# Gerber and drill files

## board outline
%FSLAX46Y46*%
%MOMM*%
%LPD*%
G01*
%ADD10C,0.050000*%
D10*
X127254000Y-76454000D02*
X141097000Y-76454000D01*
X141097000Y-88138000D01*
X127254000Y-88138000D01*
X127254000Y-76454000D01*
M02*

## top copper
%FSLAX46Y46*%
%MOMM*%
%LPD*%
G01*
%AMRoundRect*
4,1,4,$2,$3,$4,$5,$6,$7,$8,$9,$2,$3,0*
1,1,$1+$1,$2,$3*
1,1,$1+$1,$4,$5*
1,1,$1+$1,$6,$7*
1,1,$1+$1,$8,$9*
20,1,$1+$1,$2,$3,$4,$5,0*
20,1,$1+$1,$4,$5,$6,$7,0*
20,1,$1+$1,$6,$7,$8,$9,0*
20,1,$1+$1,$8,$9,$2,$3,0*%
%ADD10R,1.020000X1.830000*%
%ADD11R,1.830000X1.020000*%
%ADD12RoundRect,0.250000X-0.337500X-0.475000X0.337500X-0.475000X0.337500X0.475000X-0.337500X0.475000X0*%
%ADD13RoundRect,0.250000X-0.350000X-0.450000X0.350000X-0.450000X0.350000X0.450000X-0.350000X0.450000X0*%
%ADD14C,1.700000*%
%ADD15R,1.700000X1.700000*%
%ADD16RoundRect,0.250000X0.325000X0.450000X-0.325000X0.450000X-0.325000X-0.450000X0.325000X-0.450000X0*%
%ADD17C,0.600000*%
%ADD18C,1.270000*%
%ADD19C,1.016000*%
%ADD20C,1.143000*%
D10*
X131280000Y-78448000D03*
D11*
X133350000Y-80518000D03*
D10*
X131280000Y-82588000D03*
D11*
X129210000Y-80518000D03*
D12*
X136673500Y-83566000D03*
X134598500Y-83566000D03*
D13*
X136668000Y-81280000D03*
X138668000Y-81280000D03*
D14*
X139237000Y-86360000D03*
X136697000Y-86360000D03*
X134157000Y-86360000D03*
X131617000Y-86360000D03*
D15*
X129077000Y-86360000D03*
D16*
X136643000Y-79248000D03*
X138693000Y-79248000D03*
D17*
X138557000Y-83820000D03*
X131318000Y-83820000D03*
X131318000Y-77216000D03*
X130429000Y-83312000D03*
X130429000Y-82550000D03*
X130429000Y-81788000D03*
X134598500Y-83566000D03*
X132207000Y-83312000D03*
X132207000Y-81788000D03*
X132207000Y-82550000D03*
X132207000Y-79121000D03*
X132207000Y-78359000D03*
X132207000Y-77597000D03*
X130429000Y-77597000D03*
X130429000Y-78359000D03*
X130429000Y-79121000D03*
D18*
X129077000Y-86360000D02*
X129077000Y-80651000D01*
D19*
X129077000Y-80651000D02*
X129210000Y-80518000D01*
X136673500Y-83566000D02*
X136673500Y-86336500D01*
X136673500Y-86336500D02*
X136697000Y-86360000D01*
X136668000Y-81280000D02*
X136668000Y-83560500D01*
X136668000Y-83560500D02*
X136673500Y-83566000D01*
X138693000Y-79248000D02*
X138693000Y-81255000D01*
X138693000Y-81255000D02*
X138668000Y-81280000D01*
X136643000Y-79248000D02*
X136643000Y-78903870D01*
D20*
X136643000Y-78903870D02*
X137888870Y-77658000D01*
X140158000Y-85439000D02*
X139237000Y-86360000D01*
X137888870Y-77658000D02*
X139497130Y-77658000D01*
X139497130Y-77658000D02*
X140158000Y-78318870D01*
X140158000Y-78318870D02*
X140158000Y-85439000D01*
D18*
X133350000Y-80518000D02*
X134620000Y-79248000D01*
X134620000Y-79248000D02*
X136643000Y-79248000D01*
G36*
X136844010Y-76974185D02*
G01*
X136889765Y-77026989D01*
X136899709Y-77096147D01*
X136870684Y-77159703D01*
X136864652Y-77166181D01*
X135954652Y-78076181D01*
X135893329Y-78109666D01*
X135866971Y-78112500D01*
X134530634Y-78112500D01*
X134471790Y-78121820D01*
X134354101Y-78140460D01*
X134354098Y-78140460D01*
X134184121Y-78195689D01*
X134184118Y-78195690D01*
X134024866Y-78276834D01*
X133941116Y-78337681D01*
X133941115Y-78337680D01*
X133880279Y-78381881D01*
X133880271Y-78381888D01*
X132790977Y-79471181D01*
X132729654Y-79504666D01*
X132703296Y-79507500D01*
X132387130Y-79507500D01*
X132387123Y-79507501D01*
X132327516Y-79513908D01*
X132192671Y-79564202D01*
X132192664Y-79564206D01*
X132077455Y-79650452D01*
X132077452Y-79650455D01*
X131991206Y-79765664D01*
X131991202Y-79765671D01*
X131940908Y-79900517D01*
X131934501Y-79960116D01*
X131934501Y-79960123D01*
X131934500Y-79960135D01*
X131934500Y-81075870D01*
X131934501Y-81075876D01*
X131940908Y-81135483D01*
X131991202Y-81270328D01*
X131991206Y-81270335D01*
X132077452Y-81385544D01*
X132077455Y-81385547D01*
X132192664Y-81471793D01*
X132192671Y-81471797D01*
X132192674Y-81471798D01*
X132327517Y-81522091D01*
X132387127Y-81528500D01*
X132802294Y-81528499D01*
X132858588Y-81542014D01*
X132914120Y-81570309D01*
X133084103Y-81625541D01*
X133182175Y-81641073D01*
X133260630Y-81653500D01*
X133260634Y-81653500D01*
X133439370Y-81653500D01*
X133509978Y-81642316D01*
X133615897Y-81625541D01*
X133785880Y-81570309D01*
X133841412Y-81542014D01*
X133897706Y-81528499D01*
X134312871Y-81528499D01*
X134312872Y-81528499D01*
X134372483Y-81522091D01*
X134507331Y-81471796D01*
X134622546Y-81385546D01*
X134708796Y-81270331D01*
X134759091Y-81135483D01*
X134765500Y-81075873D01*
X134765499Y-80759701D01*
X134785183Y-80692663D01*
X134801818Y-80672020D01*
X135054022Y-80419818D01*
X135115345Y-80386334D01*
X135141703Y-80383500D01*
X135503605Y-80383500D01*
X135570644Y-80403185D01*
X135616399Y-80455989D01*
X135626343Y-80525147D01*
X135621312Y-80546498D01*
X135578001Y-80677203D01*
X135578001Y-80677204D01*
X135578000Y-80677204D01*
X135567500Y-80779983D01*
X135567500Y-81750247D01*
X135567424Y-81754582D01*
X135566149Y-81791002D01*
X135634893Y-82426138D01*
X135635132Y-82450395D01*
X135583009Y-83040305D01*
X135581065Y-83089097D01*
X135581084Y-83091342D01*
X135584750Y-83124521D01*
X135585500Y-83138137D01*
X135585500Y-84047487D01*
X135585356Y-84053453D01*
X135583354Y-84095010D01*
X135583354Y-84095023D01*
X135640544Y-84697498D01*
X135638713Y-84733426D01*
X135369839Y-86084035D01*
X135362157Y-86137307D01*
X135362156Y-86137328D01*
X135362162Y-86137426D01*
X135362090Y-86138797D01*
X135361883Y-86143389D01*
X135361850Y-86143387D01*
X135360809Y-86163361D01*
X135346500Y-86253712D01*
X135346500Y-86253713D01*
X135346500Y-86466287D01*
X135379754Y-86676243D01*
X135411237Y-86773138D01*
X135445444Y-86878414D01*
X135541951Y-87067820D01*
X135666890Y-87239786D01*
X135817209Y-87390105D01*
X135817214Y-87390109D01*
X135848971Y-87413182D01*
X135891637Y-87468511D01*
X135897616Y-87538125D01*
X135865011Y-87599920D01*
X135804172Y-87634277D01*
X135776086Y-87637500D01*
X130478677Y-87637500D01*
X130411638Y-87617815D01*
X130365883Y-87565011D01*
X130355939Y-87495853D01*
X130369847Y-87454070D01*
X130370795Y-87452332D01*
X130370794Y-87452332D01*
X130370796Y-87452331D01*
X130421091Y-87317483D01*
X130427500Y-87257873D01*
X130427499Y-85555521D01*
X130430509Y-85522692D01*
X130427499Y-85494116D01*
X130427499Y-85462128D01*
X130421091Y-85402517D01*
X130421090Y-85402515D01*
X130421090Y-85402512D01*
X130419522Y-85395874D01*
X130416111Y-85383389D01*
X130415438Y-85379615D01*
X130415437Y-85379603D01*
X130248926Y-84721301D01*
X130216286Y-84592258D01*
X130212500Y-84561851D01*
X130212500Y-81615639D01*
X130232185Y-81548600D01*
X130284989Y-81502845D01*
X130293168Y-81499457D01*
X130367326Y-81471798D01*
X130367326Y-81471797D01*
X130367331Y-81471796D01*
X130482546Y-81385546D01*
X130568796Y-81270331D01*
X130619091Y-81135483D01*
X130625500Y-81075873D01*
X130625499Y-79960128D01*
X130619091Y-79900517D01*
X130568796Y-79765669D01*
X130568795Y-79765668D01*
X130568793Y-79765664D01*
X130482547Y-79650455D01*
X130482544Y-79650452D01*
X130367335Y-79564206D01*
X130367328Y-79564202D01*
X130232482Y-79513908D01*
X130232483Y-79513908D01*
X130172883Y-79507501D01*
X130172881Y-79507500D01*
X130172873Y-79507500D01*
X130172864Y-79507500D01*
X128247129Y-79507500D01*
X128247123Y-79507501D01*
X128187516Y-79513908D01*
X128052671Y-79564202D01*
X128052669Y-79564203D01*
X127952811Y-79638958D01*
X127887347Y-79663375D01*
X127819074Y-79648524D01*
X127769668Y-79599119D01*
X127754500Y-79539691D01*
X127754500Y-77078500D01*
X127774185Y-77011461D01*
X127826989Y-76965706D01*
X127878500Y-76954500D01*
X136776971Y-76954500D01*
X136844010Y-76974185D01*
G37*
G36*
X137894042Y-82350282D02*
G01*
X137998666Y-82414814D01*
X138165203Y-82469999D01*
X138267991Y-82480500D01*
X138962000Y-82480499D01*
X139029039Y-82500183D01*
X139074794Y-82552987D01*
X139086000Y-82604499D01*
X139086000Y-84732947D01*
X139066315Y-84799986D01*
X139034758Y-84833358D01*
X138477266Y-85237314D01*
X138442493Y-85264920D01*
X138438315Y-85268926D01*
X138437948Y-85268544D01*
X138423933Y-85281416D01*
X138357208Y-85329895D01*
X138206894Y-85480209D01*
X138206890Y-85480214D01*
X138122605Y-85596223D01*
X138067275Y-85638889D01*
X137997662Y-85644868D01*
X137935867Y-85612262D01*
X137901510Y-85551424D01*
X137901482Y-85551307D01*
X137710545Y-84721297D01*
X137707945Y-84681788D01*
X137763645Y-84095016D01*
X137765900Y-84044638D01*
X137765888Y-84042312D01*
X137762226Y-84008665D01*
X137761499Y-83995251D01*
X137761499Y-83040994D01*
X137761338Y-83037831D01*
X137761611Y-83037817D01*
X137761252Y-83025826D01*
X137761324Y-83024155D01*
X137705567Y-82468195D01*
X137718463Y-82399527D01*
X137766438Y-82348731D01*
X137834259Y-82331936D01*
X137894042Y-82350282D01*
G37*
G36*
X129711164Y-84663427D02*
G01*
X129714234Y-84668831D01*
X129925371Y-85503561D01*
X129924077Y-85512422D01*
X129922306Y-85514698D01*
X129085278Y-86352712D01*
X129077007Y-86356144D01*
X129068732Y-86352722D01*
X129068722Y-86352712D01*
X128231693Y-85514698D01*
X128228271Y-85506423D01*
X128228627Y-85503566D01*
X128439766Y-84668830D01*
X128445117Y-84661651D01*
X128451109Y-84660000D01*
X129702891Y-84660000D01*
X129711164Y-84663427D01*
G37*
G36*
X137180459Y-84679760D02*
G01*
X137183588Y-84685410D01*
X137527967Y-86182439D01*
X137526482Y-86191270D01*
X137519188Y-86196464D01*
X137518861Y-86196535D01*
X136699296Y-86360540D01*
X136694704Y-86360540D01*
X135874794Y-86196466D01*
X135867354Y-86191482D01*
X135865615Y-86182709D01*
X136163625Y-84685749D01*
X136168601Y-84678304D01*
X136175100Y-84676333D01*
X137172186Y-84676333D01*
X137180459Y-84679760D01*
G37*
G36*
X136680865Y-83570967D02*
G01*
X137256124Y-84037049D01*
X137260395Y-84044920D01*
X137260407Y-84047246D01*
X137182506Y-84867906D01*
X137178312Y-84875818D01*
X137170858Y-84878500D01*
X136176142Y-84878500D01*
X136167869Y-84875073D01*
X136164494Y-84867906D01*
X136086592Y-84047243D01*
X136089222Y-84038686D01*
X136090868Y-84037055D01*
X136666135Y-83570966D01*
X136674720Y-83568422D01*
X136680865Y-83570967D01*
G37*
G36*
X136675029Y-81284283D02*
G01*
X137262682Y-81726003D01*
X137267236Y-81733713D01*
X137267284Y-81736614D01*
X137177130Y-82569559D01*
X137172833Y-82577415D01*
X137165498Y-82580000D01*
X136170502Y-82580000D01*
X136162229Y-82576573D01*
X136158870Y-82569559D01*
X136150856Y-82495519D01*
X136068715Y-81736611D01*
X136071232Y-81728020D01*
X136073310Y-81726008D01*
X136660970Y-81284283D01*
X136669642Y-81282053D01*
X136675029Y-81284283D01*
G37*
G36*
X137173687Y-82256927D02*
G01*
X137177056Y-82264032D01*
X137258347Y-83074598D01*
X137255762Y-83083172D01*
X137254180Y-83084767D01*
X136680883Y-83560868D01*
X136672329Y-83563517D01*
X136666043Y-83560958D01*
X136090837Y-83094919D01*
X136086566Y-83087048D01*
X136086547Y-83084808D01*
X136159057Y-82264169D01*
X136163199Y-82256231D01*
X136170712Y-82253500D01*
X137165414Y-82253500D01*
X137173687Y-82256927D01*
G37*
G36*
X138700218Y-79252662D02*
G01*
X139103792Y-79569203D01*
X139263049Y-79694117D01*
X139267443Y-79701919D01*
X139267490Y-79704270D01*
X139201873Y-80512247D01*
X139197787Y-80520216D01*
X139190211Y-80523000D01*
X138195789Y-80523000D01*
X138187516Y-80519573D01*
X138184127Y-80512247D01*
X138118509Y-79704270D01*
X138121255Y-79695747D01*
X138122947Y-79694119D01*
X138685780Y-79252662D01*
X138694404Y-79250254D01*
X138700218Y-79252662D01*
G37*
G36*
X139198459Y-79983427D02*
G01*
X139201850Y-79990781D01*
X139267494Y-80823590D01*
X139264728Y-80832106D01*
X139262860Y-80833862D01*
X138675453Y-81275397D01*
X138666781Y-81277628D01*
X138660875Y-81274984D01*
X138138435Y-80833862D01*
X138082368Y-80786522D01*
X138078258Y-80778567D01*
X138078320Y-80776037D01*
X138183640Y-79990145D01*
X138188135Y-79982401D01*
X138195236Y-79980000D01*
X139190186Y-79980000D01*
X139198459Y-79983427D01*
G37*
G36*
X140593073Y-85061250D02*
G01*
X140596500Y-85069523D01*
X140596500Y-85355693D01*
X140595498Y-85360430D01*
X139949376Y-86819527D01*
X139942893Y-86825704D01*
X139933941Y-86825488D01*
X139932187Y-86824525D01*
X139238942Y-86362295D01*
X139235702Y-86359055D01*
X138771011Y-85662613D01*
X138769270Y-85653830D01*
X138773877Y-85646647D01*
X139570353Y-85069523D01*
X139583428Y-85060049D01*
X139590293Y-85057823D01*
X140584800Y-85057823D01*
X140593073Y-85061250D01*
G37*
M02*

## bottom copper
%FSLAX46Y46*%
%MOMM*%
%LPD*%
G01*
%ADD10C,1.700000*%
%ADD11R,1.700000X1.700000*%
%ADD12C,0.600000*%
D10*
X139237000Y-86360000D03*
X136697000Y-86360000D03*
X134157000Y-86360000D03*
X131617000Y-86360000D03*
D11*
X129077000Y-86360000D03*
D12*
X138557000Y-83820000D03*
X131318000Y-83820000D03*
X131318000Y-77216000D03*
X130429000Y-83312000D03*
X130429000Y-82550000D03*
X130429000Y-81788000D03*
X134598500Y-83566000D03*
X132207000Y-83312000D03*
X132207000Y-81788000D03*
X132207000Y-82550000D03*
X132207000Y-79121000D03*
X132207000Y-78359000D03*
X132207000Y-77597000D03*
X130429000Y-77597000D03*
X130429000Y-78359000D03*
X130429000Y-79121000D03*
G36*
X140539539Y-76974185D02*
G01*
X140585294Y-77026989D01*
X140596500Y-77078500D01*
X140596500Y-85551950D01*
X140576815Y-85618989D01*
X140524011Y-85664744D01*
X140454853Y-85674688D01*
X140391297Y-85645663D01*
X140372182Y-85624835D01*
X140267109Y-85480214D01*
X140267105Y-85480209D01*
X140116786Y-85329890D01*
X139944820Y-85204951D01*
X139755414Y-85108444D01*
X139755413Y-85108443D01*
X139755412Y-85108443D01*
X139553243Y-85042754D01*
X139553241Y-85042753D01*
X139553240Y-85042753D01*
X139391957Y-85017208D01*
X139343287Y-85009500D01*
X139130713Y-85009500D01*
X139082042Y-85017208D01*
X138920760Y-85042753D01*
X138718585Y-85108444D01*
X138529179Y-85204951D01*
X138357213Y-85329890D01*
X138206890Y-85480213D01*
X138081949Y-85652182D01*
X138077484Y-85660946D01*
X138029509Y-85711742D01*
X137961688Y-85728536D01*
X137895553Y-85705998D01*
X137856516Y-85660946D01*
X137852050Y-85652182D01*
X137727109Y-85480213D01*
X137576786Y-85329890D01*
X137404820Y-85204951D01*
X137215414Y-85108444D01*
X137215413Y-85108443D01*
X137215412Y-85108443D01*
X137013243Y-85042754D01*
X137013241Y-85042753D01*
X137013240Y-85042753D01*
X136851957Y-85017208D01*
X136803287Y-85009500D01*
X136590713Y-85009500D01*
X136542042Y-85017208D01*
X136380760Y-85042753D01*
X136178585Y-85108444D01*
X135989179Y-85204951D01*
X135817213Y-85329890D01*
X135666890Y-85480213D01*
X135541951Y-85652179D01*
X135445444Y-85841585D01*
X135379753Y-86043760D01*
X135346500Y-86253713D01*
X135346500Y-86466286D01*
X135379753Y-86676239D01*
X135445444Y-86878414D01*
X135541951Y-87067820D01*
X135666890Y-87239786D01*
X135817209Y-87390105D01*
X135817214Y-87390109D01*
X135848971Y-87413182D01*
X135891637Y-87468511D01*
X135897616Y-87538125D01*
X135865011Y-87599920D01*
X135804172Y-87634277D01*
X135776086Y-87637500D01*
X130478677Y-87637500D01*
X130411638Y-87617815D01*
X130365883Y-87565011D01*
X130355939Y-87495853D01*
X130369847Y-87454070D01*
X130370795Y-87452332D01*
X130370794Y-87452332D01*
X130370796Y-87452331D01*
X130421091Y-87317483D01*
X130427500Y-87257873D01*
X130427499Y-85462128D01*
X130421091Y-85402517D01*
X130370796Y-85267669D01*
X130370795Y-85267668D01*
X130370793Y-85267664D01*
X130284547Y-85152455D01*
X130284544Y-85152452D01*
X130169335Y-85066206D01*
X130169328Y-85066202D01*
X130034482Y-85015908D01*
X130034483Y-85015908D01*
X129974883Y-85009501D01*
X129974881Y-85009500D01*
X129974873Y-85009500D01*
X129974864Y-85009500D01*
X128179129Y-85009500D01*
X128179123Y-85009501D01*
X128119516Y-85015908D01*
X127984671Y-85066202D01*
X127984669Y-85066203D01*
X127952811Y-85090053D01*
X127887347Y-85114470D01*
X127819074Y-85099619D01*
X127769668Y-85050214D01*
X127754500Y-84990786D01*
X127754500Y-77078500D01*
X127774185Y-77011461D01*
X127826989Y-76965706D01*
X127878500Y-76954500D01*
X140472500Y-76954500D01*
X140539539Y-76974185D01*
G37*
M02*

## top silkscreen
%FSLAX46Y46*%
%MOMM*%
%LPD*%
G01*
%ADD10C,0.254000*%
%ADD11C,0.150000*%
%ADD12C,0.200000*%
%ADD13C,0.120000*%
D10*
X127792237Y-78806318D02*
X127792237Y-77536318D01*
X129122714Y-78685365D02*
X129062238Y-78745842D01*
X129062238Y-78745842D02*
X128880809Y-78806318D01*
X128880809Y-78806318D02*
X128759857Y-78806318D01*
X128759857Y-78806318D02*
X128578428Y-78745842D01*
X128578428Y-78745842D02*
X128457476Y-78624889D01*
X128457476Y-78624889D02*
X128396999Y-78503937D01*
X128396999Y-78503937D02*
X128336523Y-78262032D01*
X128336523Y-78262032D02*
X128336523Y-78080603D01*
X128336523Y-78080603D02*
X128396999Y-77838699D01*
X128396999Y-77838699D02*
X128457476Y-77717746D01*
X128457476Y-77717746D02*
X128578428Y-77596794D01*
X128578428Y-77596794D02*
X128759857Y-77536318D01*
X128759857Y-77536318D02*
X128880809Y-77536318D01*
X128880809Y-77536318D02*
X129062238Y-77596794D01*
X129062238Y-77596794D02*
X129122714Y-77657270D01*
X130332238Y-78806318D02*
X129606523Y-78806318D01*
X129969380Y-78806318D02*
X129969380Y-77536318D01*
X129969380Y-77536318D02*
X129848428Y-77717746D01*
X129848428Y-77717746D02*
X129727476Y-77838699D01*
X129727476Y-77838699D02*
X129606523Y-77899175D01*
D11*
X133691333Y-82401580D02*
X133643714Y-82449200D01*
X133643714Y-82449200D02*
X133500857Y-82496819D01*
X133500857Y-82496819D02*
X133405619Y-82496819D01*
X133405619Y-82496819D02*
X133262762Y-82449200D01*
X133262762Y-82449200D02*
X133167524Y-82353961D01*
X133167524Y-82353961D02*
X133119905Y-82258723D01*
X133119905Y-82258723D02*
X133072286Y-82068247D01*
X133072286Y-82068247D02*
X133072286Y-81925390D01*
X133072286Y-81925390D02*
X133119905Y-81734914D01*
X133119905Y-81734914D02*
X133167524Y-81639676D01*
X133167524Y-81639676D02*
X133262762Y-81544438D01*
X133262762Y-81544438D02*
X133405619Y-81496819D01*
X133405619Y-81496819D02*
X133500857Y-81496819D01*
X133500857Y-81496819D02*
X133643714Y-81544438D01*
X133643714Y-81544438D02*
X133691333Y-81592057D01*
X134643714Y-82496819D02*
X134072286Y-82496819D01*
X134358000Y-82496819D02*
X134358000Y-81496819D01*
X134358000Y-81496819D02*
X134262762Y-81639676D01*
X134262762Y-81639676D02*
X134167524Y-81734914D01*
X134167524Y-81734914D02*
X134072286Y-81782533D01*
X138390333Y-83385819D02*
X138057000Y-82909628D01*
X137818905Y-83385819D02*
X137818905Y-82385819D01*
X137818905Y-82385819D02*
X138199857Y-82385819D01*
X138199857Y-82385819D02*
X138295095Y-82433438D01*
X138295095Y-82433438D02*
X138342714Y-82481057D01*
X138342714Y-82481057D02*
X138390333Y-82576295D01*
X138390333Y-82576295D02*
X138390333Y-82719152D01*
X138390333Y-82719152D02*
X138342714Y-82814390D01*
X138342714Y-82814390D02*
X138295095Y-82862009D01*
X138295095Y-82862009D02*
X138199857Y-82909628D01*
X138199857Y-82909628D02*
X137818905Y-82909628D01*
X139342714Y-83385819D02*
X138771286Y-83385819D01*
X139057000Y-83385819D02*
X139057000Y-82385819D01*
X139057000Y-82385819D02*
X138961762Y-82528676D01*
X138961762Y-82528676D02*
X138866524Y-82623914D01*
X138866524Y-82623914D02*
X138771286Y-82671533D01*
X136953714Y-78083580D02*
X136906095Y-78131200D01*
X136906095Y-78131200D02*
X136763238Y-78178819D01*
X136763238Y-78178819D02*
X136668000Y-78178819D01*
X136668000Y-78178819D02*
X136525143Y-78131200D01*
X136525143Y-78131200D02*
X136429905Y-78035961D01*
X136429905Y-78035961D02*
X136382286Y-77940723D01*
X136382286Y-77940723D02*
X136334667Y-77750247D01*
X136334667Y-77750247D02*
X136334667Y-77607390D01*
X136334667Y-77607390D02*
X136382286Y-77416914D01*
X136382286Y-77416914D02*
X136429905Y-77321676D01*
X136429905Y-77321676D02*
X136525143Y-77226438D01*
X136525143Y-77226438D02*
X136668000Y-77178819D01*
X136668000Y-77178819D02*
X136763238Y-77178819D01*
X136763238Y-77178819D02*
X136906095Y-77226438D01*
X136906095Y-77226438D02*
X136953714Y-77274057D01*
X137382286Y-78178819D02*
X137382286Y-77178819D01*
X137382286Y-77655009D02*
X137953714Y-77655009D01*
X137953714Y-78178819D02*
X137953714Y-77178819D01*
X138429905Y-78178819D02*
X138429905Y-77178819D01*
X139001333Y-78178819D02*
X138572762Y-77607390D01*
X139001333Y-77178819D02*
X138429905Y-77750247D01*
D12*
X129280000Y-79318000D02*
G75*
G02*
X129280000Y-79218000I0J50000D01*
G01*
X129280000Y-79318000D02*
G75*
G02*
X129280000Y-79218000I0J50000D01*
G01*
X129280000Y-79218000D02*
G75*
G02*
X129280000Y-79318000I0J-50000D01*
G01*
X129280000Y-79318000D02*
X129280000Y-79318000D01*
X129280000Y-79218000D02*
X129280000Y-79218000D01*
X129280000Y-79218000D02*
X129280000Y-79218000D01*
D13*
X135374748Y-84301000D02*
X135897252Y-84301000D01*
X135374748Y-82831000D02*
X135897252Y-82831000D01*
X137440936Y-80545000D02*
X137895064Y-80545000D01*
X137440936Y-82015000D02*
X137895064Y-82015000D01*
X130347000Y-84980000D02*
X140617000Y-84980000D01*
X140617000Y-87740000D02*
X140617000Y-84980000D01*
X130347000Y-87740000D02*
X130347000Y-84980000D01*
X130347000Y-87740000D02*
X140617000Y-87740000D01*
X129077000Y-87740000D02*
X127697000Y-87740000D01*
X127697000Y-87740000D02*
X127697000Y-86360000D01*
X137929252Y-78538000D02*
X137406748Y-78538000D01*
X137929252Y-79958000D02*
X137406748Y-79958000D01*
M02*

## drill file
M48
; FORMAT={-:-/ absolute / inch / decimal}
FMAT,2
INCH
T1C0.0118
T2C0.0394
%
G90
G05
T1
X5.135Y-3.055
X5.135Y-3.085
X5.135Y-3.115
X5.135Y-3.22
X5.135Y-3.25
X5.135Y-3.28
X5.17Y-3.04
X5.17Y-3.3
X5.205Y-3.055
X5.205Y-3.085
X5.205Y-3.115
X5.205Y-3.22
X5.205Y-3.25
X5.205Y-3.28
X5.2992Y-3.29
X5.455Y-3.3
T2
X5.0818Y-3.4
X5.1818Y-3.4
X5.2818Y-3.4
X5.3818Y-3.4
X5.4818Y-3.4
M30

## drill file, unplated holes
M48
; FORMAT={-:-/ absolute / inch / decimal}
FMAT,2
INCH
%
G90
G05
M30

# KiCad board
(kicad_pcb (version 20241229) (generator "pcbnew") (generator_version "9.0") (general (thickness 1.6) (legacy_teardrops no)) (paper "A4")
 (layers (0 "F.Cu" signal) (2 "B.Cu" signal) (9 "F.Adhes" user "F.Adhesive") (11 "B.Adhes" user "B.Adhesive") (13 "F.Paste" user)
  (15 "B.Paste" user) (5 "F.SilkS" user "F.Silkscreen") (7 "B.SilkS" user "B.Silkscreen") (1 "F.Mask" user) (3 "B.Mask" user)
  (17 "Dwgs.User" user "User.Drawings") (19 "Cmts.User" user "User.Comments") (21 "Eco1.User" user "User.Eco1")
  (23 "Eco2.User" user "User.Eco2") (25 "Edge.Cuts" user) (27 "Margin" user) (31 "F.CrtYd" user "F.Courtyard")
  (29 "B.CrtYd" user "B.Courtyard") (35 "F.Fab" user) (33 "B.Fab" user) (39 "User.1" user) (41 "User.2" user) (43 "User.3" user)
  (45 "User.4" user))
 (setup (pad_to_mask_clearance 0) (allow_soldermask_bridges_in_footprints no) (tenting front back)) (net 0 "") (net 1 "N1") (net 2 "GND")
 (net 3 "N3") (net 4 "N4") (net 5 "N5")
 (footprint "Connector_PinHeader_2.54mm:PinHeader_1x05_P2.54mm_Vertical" (layer "F.Cu") (at 129.077 86.36 90)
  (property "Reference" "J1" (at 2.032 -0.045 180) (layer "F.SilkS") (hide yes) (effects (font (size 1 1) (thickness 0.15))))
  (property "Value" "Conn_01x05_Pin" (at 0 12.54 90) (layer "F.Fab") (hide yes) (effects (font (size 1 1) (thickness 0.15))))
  (fp_line (start -1.38 -1.38) (end 0 -1.38) (stroke (width 0.12) (type solid)) (layer "F.SilkS"))
  (fp_line (start -1.38 0) (end -1.38 -1.38) (stroke (width 0.12) (type solid)) (layer "F.SilkS"))
  (fp_line (start 1.38 1.27) (end 1.38 11.54) (stroke (width 0.12) (type solid)) (layer "F.SilkS"))
  (fp_line (start -1.38 1.27) (end 1.38 1.27) (stroke (width 0.12) (type solid)) (layer "F.SilkS"))
  (fp_line (start -1.38 1.27) (end -1.38 11.54) (stroke (width 0.12) (type solid)) (layer "F.SilkS"))
  (fp_line (start -1.38 11.54) (end 1.38 11.54) (stroke (width 0.12) (type solid)) (layer "F.SilkS"))
  (pad "1" thru_hole rect (at 0 0 90) (size 1.7 1.7) (drill 1) (layers "*.Cu" "*.Mask") (remove_unused_layers no) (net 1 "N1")
   (teardrops (best_length_ratio 0.5) (max_length 1) (best_width_ratio 1) (max_width 2) (curved_edges no) (filter_ratio 0.9) (enabled yes)
    (allow_two_segments yes) (prefer_zone_connections yes)))
  (pad "2" thru_hole circle (at 0 2.54 90) (size 1.7 1.7) (drill 1) (layers "*.Cu" "*.Mask") (remove_unused_layers no) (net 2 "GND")
   (zone_connect 2))
  (pad "3" thru_hole circle (at 0 5.08 90) (size 1.7 1.7) (drill 1) (layers "*.Cu" "*.Mask") (remove_unused_layers no) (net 2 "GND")
   (zone_connect 2))
  (pad "4" thru_hole circle (at 0 7.62 90) (size 1.7 1.7) (drill 1) (layers "*.Cu" "*.Mask") (remove_unused_layers no) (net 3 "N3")
   (teardrops (best_length_ratio 0.5) (max_length 1) (best_width_ratio 1) (max_width 2) (curved_edges no) (filter_ratio 0.9) (enabled yes)
    (allow_two_segments yes) (prefer_zone_connections yes)))
  (pad "5" thru_hole circle (at 0 10.16 90) (size 1.7 1.7) (drill 1) (layers "*.Cu" "*.Mask") (remove_unused_layers no) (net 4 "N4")
   (teardrops (best_length_ratio 0.5) (max_length 1) (best_width_ratio 1) (max_width 2) (curved_edges no) (filter_ratio 0.9) (enabled yes)
    (allow_two_segments yes) (prefer_zone_connections yes))))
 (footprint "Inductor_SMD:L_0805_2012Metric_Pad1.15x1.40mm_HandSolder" (layer "F.Cu") (at 137.668 79.248 180)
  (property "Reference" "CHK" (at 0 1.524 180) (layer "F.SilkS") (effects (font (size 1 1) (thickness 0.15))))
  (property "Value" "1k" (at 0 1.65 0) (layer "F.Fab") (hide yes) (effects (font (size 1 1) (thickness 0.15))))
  (fp_line (start -0.261252 0.71) (end 0.261252 0.71) (stroke (width 0.12) (type solid)) (layer "F.SilkS"))
  (fp_line (start -0.261252 -0.71) (end 0.261252 -0.71) (stroke (width 0.12) (type solid)) (layer "F.SilkS"))
  (pad "1" smd roundrect (at -1.025 0 180) (size 1.15 1.4) (layers "F.Cu" "F.Mask" "F.Paste") (roundrect_rratio 0.217391) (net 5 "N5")
   (teardrops (best_length_ratio 0.5) (max_length 1) (best_width_ratio 1) (max_width 2) (curved_edges no) (filter_ratio 0.9) (enabled yes)
    (allow_two_segments yes) (prefer_zone_connections yes)))
  (pad "2" smd roundrect (at 1.025 0 180) (size 1.15 1.4) (layers "F.Cu" "F.Mask" "F.Paste") (roundrect_rratio 0.217391) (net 4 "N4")
   (teardrops (best_length_ratio 0.5) (max_length 1) (best_width_ratio 1) (max_width 2) (curved_edges no) (filter_ratio 0.9) (enabled yes)
    (allow_two_segments yes) (prefer_zone_connections yes))))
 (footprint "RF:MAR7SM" (layer "F.Cu") (at 131.28 80.518 -90)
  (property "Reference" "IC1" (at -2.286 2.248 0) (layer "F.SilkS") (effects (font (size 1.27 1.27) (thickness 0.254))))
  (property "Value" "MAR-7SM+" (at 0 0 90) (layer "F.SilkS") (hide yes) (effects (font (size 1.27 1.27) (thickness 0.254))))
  (fp_line (start -1.3 2) (end -1.3 2) (stroke (width 0.2) (type solid)) (layer "F.SilkS"))
  (fp_line (start -1.3 2) (end -1.3 2) (stroke (width 0.2) (type solid)) (layer "F.SilkS"))
  (fp_line (start -1.2 2) (end -1.2 2) (stroke (width 0.2) (type solid)) (layer "F.SilkS"))
  (fp_arc (start -1.3 2) (mid -1.25 1.95) (end -1.2 2) (stroke (width 0.2) (type solid)) (layer "F.SilkS"))
  (fp_arc (start -1.2 2) (mid -1.25 2.05) (end -1.3 2) (stroke (width 0.2) (type solid)) (layer "F.SilkS"))
  (fp_arc (start -1.2 2) (mid -1.25 2.05) (end -1.3 2) (stroke (width 0.2) (type solid)) (layer "F.SilkS"))
  (pad "1" smd rect (at 0 2.07 270) (size 1.02 1.83) (layers "F.Cu" "F.Mask" "F.Paste") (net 1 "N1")
   (teardrops (best_length_ratio 0.5) (max_length 1) (best_width_ratio 1) (max_width 2) (curved_edges no) (filter_ratio 0.9) (enabled yes)
    (allow_two_segments yes) (prefer_zone_connections yes)))
  (pad "2" smd rect (at 2.07 0) (size 1.02 1.83) (layers "F.Cu" "F.Mask" "F.Paste") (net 2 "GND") (zone_connect 2))
  (pad "3" smd rect (at 0 -2.07 270) (size 1.02 1.83) (layers "F.Cu" "F.Mask" "F.Paste") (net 4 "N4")
   (teardrops (best_length_ratio 0.5) (max_length 1) (best_width_ratio 1) (max_width 2) (curved_edges no) (filter_ratio 0.9) (enabled yes)
    (allow_two_segments yes) (prefer_zone_connections yes)))
  (pad "4" smd rect (at -2.07 0) (size 1.02 1.83) (layers "F.Cu" "F.Mask" "F.Paste") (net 2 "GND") (zone_connect 2)))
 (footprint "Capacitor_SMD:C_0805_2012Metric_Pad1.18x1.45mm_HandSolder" (layer "F.Cu") (at 135.636 83.566)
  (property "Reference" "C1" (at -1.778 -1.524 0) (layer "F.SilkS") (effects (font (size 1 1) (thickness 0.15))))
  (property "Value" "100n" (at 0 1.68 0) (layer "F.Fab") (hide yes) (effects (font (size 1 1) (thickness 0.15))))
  (fp_line (start -0.261252 -0.735) (end 0.261252 -0.735) (stroke (width 0.12) (type solid)) (layer "F.SilkS"))
  (fp_line (start -0.261252 0.735) (end 0.261252 0.735) (stroke (width 0.12) (type solid)) (layer "F.SilkS"))
  (pad "1" smd roundrect (at -1.0375 0) (size 1.175 1.45) (layers "F.Cu" "F.Mask" "F.Paste") (roundrect_rratio 0.212766) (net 2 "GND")
   (zone_connect 2))
  (pad "2" smd roundrect (at 1.0375 0) (size 1.175 1.45) (layers "F.Cu" "F.Mask" "F.Paste") (roundrect_rratio 0.212766) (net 3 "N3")
   (teardrops (best_length_ratio 0.5) (max_length 1) (best_width_ratio 1) (max_width 2) (curved_edges no) (filter_ratio 0.9) (enabled yes)
    (allow_two_segments yes) (prefer_zone_connections yes))))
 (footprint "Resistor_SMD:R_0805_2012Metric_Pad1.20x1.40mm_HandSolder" (layer "F.Cu") (at 137.668 81.28)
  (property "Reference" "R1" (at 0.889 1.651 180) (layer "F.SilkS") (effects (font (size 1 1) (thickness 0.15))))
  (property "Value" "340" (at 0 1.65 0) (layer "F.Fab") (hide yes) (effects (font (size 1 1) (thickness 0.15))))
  (fp_line (start -0.227064 -0.735) (end 0.227064 -0.735) (stroke (width 0.12) (type solid)) (layer "F.SilkS"))
  (fp_line (start -0.227064 0.735) (end 0.227064 0.735) (stroke (width 0.12) (type solid)) (layer "F.SilkS"))
  (pad "1" smd roundrect (at -1 0) (size 1.2 1.4) (layers "F.Cu" "F.Mask" "F.Paste") (roundrect_rratio 0.208333) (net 3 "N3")
   (teardrops (best_length_ratio 0.5) (max_length 1) (best_width_ratio 1) (max_width 2) (curved_edges no) (filter_ratio 0.9) (enabled yes)
    (allow_two_segments yes) (prefer_zone_connections yes)))
  (pad "2" smd roundrect (at 1 0) (size 1.2 1.4) (layers "F.Cu" "F.Mask" "F.Paste") (roundrect_rratio 0.208333) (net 5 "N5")
   (teardrops (best_length_ratio 0.5) (max_length 1) (best_width_ratio 1) (max_width 2) (curved_edges no) (filter_ratio 0.9) (enabled yes)
    (allow_two_segments yes) (prefer_zone_connections yes))))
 (gr_rect (start 127.254 76.454) (end 141.097 88.138) (stroke (width 0.05) (type default)) (fill no) (layer "Edge.Cuts"))
 (segment (start 139.49713 77.658) (end 140.158 78.31887) (width 1.143) (layer "F.Cu") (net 4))
 (segment (start 133.35 80.518) (end 134.62 79.248) (width 1.27) (layer "F.Cu") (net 4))
 (segment (start 137.88887 77.658) (end 139.49713 77.658) (width 1.143) (layer "F.Cu") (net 4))
 (segment (start 134.62 79.248) (end 136.643 79.248) (width 1.27) (layer "F.Cu") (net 4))
 (segment (start 136.643 79.248) (end 136.643 78.90387) (width 1.016) (layer "F.Cu") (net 4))
 (segment (start 140.158 85.439) (end 139.237 86.36) (width 1.143) (layer "F.Cu") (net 4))
 (segment (start 136.643 78.90387) (end 137.88887 77.658) (width 1.143) (layer "F.Cu") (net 4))
 (segment (start 140.158 78.31887) (end 140.158 85.439) (width 1.143) (layer "F.Cu") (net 4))
 (segment (start 138.693 79.248) (end 138.693 81.255) (width 1.016) (layer "F.Cu") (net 5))
 (segment (start 138.693 81.255) (end 138.668 81.28) (width 1.016) (layer "F.Cu") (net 5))
 (segment (start 129.077 80.651) (end 129.21 80.518) (width 1.016) (layer "F.Cu") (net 1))
 (segment (start 129.077 86.36) (end 129.077 80.651) (width 1.27) (layer "F.Cu") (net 1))
 (via (at 132.207 78.359) (size 0.6) (drill 0.3) (layers "F.Cu" "B.Cu") (free yes) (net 2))
 (via (at 134.5985 83.566) (size 0.6) (drill 0.3) (layers "F.Cu" "B.Cu") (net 2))
 (via (at 130.429 79.121) (size 0.6) (drill 0.3) (layers "F.Cu" "B.Cu") (free yes) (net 2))
 (via (at 130.429 83.312) (size 0.6) (drill 0.3) (layers "F.Cu" "B.Cu") (free yes) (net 2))
 (via (at 131.318 77.216) (size 0.6) (drill 0.3) (layers "F.Cu" "B.Cu") (free yes) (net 2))
 (via (at 130.429 77.597) (size 0.6) (drill 0.3) (layers "F.Cu" "B.Cu") (free yes) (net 2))
 (via (at 130.429 81.788) (size 0.6) (drill 0.3) (layers "F.Cu" "B.Cu") (free yes) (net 2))
 (via (at 138.557 83.82) (size 0.6) (drill 0.3) (layers "F.Cu" "B.Cu") (free yes) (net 2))
 (via (at 132.207 79.121) (size 0.6) (drill 0.3) (layers "F.Cu" "B.Cu") (free yes) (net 2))
 (via (at 132.207 83.312) (size 0.6) (drill 0.3) (layers "F.Cu" "B.Cu") (free yes) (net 2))
 (via (at 130.429 78.359) (size 0.6) (drill 0.3) (layers "F.Cu" "B.Cu") (free yes) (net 2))
 (via (at 132.207 82.55) (size 0.6) (drill 0.3) (layers "F.Cu" "B.Cu") (free yes) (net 2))
 (via (at 132.207 81.788) (size 0.6) (drill 0.3) (layers "F.Cu" "B.Cu") (free yes) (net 2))
 (via (at 130.429 82.55) (size 0.6) (drill 0.3) (layers "F.Cu" "B.Cu") (free yes) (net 2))
 (via (at 131.318 83.82) (size 0.6) (drill 0.3) (layers "F.Cu" "B.Cu") (free yes) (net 2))
 (via (at 132.207 77.597) (size 0.6) (drill 0.3) (layers "F.Cu" "B.Cu") (free yes) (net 2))
 (segment (start 136.6735 83.566) (end 136.6735 86.3365) (width 1.016) (layer "F.Cu") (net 3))
 (segment (start 136.668 83.5605) (end 136.6735 83.566) (width 1.016) (layer "F.Cu") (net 3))
 (segment (start 136.6735 86.3365) (end 136.697 86.36) (width 1.016) (layer "F.Cu") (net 3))
 (segment (start 136.668 81.28) (end 136.668 83.5605) (width 1.016) (layer "F.Cu") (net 3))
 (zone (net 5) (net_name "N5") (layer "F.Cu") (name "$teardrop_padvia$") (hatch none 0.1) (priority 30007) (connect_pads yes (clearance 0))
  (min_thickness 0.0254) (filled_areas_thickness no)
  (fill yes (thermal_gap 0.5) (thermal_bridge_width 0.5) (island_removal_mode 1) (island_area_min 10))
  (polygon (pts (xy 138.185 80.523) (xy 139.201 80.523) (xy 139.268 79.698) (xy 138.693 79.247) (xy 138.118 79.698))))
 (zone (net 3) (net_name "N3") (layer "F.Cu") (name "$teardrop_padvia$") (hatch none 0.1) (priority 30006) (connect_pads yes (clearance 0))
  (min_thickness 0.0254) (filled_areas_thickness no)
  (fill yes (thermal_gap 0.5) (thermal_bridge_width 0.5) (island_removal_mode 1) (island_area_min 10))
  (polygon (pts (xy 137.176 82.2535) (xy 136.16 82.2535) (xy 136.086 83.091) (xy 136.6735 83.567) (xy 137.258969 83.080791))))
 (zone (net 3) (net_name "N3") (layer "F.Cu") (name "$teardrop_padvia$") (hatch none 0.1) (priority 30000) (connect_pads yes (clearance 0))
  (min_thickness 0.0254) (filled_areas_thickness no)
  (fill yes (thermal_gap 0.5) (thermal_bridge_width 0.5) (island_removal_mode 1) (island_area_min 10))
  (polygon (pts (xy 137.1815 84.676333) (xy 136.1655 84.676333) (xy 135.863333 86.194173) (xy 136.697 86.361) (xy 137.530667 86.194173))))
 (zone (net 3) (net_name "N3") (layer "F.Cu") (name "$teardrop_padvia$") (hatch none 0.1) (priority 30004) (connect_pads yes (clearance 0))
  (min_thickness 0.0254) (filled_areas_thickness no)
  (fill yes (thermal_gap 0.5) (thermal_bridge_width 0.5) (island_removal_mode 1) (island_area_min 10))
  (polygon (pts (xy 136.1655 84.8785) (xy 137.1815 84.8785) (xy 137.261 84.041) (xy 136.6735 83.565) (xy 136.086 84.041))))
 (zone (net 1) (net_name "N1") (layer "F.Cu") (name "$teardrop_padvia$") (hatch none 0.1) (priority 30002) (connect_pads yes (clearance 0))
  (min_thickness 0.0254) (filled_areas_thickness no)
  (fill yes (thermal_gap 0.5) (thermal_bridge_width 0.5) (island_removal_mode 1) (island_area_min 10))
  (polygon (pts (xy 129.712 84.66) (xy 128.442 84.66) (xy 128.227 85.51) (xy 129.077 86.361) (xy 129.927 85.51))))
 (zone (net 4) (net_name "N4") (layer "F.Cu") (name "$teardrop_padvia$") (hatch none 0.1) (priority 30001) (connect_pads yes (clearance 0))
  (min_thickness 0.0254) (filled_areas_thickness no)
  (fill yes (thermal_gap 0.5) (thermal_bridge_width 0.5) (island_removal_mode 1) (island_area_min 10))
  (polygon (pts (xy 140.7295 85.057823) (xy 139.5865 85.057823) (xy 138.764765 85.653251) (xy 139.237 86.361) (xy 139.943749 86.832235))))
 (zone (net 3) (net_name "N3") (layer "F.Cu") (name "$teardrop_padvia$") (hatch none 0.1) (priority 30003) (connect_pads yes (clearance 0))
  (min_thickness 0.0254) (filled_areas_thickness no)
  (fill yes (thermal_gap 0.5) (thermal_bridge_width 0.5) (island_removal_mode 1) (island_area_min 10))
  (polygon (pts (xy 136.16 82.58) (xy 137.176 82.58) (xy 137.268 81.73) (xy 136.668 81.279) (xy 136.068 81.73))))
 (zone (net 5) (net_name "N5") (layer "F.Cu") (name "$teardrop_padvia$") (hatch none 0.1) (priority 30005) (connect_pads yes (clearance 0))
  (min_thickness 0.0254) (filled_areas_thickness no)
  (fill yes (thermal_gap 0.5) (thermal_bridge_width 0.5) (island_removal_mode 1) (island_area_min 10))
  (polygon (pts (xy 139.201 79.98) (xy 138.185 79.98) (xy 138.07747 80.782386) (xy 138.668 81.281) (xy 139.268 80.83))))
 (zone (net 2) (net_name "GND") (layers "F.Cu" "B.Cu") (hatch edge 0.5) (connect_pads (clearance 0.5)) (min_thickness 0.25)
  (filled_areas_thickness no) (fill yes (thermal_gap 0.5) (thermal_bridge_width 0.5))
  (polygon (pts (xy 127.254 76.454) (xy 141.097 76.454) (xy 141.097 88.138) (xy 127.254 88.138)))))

